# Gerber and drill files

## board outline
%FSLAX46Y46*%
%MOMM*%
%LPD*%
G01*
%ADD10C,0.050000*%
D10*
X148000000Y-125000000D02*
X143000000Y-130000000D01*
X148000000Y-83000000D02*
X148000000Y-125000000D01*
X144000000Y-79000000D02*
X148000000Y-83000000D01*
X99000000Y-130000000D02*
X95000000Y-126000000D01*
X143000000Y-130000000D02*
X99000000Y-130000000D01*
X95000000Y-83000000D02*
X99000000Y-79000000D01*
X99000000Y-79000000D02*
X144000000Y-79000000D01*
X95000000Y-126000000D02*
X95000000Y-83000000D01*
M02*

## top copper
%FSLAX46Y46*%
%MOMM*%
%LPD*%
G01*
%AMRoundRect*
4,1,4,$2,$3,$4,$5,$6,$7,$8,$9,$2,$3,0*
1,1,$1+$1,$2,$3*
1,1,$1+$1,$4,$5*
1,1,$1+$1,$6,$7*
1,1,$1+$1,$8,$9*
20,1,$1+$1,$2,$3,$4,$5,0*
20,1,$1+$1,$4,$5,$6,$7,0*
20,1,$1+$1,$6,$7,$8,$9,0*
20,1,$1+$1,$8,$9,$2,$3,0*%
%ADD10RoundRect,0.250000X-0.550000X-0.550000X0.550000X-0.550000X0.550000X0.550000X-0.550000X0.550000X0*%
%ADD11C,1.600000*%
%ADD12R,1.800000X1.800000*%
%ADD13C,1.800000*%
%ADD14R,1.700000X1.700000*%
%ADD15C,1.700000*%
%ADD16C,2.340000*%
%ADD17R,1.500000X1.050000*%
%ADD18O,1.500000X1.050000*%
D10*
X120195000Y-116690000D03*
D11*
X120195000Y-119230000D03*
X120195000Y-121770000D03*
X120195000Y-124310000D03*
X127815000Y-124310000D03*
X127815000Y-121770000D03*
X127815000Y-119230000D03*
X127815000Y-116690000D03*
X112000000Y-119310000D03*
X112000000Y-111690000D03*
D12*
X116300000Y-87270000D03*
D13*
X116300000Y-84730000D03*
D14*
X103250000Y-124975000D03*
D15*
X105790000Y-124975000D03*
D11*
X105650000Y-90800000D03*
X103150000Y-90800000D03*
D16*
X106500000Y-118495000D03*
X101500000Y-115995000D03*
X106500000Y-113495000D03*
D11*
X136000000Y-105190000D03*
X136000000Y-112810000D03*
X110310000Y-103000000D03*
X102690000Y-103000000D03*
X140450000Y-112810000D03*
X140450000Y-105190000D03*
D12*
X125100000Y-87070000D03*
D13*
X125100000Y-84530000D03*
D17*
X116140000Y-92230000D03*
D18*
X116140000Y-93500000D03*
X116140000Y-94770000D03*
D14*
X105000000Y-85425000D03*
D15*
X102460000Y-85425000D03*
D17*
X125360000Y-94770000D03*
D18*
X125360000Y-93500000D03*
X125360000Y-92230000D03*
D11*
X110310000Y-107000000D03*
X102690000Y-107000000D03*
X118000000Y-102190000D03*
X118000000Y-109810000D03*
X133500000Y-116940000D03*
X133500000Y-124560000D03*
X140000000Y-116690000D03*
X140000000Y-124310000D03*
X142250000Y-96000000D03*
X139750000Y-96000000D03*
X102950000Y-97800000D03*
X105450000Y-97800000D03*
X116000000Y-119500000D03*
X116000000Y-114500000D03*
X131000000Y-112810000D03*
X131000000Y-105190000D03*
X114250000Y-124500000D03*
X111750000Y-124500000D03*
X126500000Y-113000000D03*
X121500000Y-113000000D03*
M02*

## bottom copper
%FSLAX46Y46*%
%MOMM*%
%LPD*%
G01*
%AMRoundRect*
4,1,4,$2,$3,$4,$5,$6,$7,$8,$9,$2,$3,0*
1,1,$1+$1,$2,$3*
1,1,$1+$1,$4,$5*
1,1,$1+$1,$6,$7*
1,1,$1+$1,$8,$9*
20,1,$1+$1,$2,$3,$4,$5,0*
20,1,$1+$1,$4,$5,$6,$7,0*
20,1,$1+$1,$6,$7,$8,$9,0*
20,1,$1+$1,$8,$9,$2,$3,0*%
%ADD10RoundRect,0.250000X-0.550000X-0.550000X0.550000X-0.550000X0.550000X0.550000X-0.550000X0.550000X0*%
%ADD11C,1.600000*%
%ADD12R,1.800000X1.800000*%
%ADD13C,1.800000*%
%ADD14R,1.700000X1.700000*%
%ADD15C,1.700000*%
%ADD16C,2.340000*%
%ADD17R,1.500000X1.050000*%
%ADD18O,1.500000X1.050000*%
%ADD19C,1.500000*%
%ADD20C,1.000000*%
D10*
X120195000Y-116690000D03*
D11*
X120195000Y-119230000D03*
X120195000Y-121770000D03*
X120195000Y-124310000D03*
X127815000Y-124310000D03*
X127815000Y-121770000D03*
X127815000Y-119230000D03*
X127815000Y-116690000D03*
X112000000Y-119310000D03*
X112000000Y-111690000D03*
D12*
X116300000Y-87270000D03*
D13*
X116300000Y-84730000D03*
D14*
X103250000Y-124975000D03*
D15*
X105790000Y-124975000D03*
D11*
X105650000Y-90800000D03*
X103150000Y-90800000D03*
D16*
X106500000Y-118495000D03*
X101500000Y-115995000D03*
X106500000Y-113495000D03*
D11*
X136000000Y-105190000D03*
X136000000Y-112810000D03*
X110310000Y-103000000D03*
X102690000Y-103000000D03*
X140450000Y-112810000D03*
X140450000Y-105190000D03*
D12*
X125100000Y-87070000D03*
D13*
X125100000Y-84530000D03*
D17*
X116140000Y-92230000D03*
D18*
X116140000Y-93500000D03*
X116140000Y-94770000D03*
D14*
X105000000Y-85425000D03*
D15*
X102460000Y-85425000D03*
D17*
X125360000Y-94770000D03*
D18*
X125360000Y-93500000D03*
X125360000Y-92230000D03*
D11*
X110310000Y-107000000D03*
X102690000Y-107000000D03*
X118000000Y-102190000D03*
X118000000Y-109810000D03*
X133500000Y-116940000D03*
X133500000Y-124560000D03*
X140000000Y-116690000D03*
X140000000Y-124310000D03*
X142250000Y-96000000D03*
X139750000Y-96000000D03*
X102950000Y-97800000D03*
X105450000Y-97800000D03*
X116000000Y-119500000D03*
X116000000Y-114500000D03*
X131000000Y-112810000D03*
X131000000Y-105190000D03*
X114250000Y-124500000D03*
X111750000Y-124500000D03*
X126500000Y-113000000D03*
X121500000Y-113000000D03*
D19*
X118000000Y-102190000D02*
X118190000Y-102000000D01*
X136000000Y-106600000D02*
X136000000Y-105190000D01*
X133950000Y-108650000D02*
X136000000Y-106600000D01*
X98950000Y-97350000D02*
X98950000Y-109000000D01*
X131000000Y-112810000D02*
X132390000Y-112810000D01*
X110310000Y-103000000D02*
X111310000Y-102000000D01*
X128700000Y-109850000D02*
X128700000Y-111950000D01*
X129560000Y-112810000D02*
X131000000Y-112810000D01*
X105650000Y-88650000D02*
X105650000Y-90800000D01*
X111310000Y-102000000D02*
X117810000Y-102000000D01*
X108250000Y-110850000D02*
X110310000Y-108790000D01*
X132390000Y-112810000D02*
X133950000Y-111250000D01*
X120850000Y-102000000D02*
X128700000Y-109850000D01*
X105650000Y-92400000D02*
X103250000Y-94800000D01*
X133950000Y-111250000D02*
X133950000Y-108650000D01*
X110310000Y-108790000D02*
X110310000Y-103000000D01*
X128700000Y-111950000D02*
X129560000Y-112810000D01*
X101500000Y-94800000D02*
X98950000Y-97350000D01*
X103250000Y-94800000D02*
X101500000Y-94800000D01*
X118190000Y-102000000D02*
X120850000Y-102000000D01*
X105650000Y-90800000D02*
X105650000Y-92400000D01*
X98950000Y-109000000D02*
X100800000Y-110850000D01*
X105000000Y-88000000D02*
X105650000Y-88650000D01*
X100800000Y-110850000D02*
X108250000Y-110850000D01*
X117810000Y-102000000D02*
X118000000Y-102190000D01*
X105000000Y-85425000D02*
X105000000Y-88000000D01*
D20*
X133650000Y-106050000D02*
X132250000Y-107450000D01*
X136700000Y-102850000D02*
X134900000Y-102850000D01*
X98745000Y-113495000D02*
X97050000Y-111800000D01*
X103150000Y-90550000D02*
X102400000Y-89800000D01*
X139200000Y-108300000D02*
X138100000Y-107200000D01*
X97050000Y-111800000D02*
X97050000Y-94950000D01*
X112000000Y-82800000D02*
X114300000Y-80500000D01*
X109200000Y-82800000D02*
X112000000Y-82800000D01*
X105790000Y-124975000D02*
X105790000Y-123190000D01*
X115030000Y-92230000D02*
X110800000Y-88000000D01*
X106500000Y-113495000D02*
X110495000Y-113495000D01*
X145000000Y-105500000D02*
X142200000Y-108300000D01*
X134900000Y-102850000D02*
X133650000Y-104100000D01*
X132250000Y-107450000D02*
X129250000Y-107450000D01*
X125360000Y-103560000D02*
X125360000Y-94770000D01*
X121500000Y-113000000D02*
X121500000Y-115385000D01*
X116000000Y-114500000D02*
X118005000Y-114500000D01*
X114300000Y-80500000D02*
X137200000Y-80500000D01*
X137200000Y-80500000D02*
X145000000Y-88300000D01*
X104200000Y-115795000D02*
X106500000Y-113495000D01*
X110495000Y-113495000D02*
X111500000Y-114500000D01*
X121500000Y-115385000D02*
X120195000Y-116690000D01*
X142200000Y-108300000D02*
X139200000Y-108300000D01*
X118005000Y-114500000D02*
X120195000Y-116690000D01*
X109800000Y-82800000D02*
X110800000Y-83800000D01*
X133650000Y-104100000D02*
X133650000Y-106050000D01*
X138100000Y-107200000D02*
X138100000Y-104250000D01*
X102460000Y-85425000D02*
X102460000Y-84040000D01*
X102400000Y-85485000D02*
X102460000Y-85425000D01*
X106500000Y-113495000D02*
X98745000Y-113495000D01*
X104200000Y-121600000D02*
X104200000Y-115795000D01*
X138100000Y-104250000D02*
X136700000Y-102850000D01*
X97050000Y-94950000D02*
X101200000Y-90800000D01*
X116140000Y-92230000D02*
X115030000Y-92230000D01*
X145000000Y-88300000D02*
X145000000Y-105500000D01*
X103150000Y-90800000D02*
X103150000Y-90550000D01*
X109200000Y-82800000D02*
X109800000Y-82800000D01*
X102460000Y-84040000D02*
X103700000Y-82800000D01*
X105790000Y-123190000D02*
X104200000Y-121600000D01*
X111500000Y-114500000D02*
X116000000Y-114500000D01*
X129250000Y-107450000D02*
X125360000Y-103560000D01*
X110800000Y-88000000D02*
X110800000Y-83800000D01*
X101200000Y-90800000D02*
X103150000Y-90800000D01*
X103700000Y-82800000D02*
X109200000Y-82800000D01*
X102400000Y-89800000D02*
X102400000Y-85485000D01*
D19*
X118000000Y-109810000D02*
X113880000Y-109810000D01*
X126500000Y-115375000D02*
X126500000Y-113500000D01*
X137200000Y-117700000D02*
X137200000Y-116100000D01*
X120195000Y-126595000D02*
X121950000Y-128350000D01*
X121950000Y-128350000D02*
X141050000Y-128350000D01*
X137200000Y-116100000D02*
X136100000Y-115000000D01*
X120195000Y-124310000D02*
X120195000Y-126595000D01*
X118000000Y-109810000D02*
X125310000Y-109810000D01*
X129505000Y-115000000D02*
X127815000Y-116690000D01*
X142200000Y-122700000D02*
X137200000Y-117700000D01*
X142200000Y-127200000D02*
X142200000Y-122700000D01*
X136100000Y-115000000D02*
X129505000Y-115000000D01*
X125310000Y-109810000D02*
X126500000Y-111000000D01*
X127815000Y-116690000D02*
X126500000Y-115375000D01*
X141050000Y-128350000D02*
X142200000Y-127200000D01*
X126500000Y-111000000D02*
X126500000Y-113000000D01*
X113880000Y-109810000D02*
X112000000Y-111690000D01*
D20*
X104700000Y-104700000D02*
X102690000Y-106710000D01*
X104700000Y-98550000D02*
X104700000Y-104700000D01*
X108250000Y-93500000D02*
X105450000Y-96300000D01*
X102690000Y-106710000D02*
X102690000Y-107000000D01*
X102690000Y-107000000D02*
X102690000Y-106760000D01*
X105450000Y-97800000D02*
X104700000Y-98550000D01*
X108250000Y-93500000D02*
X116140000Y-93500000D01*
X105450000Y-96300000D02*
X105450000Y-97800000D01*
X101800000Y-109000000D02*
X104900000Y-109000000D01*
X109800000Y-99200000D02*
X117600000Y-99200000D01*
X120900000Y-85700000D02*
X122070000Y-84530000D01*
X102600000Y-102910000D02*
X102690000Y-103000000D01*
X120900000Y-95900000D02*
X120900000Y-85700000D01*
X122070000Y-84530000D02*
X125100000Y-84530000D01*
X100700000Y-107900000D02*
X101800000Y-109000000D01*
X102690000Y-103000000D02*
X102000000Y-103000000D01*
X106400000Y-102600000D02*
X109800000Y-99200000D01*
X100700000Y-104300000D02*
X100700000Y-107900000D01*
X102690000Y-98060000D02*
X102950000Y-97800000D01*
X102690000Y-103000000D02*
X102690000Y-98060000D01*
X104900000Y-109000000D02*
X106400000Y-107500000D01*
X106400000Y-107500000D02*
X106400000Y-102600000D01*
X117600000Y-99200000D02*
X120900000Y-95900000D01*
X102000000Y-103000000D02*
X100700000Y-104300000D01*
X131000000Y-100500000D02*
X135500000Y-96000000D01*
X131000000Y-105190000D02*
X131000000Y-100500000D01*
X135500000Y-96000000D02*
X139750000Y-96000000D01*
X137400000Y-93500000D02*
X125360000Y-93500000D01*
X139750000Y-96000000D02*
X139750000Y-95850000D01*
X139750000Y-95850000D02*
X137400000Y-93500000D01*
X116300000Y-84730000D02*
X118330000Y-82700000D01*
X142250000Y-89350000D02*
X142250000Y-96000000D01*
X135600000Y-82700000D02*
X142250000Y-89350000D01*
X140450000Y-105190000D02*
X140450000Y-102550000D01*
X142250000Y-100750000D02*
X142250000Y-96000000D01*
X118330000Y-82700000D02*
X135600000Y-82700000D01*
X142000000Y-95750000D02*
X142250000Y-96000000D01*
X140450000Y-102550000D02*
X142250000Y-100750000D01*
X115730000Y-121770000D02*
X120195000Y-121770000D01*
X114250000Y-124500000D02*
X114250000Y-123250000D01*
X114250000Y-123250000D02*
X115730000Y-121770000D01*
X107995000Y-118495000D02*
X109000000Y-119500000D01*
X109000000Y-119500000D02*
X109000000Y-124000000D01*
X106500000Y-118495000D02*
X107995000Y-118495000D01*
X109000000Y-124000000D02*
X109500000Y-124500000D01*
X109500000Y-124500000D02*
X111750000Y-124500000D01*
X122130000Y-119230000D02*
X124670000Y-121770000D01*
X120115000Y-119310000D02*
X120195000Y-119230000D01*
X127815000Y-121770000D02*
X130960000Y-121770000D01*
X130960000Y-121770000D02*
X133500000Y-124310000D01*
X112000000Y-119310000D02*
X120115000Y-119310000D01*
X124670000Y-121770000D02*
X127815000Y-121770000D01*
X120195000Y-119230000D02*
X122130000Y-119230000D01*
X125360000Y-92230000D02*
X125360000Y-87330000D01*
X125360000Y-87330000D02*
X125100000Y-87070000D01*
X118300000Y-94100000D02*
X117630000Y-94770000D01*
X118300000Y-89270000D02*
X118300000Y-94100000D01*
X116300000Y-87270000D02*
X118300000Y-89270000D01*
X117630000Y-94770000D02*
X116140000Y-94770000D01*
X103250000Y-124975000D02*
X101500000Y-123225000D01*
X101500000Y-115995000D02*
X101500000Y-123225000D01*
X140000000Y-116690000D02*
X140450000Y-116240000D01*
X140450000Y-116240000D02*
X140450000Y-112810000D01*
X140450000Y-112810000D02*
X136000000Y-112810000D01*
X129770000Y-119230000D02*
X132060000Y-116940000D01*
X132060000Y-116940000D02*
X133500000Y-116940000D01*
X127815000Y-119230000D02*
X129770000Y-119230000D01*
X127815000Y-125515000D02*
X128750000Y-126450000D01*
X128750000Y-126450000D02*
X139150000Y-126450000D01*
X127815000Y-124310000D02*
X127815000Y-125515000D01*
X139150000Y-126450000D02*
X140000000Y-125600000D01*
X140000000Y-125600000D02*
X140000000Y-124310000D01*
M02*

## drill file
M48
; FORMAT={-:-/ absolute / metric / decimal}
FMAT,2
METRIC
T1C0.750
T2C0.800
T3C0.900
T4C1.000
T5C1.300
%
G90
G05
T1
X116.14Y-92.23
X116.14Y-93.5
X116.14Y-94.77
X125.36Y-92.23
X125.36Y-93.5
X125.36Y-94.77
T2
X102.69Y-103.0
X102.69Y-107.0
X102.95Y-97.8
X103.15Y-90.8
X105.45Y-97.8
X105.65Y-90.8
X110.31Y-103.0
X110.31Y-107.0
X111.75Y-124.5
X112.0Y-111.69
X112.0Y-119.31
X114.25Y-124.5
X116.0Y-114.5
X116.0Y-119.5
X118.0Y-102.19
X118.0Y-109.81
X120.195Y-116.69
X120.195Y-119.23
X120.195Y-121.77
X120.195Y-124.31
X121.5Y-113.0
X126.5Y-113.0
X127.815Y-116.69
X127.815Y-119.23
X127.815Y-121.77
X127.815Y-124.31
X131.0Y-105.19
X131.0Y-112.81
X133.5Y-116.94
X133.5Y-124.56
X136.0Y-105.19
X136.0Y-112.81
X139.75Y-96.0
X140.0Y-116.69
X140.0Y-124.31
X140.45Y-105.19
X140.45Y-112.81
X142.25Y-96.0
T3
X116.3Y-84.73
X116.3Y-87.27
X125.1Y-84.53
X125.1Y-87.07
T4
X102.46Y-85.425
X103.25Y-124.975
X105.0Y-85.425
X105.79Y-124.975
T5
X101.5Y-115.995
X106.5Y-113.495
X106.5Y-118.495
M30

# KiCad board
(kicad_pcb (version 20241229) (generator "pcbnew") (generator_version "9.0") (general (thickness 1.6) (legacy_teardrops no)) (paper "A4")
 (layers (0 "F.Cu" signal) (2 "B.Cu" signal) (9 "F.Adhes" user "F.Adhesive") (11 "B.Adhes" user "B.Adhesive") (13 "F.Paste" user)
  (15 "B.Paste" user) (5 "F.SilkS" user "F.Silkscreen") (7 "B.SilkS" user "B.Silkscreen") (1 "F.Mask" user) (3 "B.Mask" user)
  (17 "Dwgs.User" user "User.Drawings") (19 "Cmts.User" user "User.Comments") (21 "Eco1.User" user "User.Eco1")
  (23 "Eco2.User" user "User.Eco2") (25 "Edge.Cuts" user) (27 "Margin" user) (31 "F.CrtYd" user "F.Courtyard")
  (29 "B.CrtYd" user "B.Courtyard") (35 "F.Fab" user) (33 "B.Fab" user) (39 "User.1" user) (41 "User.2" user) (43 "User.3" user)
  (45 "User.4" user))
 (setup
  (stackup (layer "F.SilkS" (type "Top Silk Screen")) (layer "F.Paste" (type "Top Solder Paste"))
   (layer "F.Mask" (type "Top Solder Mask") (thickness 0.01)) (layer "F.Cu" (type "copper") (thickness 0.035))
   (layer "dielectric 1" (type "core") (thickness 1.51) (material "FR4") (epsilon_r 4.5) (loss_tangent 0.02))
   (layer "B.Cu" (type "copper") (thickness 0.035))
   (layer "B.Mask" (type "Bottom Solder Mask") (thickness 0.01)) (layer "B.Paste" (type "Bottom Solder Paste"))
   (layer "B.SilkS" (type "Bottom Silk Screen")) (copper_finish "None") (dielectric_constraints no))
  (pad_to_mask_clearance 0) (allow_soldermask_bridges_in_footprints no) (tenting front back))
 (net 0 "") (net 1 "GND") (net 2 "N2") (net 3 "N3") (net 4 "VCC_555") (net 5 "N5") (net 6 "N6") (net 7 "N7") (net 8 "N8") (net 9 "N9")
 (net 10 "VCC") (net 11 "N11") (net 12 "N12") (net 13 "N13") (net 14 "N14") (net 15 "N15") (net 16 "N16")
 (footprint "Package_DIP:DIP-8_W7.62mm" (layer "F.Cu") (at 120.195 116.69)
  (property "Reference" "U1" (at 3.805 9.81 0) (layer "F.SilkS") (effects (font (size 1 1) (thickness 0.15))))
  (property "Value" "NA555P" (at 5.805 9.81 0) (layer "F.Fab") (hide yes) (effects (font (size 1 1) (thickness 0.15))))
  (pad "1" thru_hole roundrect (at 0 0) (size 1.6 1.6) (drill 0.8) (layers "*.Cu" "*.Mask") (remove_unused_layers no)
   (roundrect_rratio 0.15625) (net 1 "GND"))
  (pad "2" thru_hole circle (at 0 2.54) (size 1.6 1.6) (drill 0.8) (layers "*.Cu" "*.Mask") (remove_unused_layers no) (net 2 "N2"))
  (pad "3" thru_hole circle (at 0 5.08) (size 1.6 1.6) (drill 0.8) (layers "*.Cu" "*.Mask") (remove_unused_layers no) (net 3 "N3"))
  (pad "4" thru_hole circle (at 0 7.62) (size 1.6 1.6) (drill 0.8) (layers "*.Cu" "*.Mask") (remove_unused_layers no) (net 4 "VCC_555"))
  (pad "5" thru_hole circle (at 7.62 7.62) (size 1.6 1.6) (drill 0.8) (layers "*.Cu" "*.Mask") (remove_unused_layers no) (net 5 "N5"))
  (pad "6" thru_hole circle (at 7.62 5.08) (size 1.6 1.6) (drill 0.8) (layers "*.Cu" "*.Mask") (remove_unused_layers no) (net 2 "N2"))
  (pad "7" thru_hole circle (at 7.62 2.54) (size 1.6 1.6) (drill 0.8) (layers "*.Cu" "*.Mask") (remove_unused_layers no) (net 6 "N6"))
  (pad "8" thru_hole circle (at 7.62 0) (size 1.6 1.6) (drill 0.8) (layers "*.Cu" "*.Mask") (remove_unused_layers no) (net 4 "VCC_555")))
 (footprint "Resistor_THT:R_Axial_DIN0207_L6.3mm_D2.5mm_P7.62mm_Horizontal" (layer "F.Cu") (at 112 119.31 90)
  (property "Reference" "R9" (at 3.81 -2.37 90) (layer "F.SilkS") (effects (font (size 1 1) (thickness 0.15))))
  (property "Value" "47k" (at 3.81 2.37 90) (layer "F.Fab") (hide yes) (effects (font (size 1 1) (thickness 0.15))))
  (pad "1" thru_hole circle (at 0 0 90) (size 1.6 1.6) (drill 0.8) (layers "*.Cu" "*.Mask") (remove_unused_layers no) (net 2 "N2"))
  (pad "2" thru_hole circle (at 7.62 0 90) (size 1.6 1.6) (drill 0.8) (layers "*.Cu" "*.Mask") (remove_unused_layers no) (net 4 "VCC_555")))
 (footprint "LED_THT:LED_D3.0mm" (layer "F.Cu") (at 116.3 87.27 90)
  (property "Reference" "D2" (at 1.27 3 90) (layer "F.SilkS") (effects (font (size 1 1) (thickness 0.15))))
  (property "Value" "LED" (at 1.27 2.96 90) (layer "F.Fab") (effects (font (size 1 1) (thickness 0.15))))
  (pad "1" thru_hole rect (at 0 0 90) (size 1.8 1.8) (drill 0.9) (layers "*.Cu" "*.Mask") (remove_unused_layers no) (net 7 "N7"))
  (pad "2" thru_hole circle (at 2.54 0 90) (size 1.8 1.8) (drill 0.9) (layers "*.Cu" "*.Mask") (remove_unused_layers no) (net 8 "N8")))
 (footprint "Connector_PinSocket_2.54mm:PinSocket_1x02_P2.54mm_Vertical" (layer "F.Cu") (at 103.25 124.975 90)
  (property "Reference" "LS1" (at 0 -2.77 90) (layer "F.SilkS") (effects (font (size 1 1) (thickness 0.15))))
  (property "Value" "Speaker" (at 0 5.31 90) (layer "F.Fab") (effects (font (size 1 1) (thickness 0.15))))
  (pad "1" thru_hole rect (at 0 0 90) (size 1.7 1.7) (drill 1) (layers "*.Cu" "*.Mask") (remove_unused_layers no) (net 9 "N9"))
  (pad "2" thru_hole circle (at 0 2.54 90) (size 1.7 1.7) (drill 1) (layers "*.Cu" "*.Mask") (remove_unused_layers no) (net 1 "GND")))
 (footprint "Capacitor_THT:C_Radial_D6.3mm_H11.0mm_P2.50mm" (layer "F.Cu") (at 105.65 90.8 180)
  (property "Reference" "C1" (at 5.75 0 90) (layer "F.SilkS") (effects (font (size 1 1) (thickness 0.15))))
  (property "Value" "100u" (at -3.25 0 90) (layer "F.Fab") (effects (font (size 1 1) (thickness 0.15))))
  (pad "1" thru_hole circle (at 0 0 180) (size 1.6 1.6) (drill 0.8) (layers "*.Cu" "*.Mask") (remove_unused_layers no) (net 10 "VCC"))
  (pad "2" thru_hole circle (at 2.5 0 180) (size 1.6 1.6) (drill 0.8) (layers "*.Cu" "*.Mask") (remove_unused_layers no) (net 1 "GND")))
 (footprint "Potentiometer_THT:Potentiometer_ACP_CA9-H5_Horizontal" (layer "F.Cu") (at 106.5 118.495 180)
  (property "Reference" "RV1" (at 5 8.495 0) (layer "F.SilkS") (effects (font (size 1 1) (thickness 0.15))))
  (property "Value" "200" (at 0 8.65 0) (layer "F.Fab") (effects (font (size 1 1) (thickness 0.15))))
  (pad "1" thru_hole circle (at 0 0 180) (size 2.34 2.34) (drill 1.3) (layers "*.Cu" "*.Mask") (remove_unused_layers no) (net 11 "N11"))
  (pad "2" thru_hole circle (at 5 2.5 180) (size 2.34 2.34) (drill 1.3) (layers "*.Cu" "*.Mask") (remove_unused_layers no) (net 9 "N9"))
  (pad "3" thru_hole circle (at 0 5 180) (size 2.34 2.34) (drill 1.3) (layers "*.Cu" "*.Mask") (remove_unused_layers no) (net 1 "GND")))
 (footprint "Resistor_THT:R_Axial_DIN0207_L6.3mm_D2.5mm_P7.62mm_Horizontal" (layer "F.Cu") (at 136 105.19 -90)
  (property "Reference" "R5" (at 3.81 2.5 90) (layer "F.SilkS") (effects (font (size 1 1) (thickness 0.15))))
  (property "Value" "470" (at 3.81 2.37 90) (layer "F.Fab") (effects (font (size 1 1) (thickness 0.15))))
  (pad "1" thru_hole circle (at 0 0 270) (size 1.6 1.6) (drill 0.8) (layers "*.Cu" "*.Mask") (remove_unused_layers no) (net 10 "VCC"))
  (pad "2" thru_hole circle (at 7.62 0 270) (size 1.6 1.6) (drill 0.8) (layers "*.Cu" "*.Mask") (remove_unused_layers no) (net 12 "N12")))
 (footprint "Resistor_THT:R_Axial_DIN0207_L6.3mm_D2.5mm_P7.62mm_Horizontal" (layer "F.Cu") (at 110.31 103 180)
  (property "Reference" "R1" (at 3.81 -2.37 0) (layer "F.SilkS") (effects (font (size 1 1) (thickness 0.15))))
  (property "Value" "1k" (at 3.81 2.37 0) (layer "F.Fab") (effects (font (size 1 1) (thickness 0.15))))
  (pad "1" thru_hole circle (at 0 0 180) (size 1.6 1.6) (drill 0.8) (layers "*.Cu" "*.Mask") (remove_unused_layers no) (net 10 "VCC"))
  (pad "2" thru_hole circle (at 7.62 0 180) (size 1.6 1.6) (drill 0.8) (layers "*.Cu" "*.Mask") (remove_unused_layers no) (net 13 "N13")))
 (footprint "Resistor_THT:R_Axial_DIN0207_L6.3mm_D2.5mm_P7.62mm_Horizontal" (layer "F.Cu") (at 140.45 112.81 90)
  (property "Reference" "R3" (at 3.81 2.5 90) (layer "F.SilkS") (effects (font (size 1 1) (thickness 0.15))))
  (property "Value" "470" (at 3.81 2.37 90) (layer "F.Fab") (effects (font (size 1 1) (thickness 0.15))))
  (pad "1" thru_hole circle (at 0 0 90) (size 1.6 1.6) (drill 0.8) (layers "*.Cu" "*.Mask") (remove_unused_layers no) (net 12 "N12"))
  (pad "2" thru_hole circle (at 7.62 0 90) (size 1.6 1.6) (drill 0.8) (layers "*.Cu" "*.Mask") (remove_unused_layers no) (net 8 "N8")))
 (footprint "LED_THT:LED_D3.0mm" (layer "F.Cu") (at 125.1 87.07 90)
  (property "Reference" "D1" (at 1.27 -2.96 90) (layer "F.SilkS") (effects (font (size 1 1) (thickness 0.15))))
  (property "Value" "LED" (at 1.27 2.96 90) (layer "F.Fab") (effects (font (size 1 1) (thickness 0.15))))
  (pad "1" thru_hole rect (at 0 0 90) (size 1.8 1.8) (drill 0.9) (layers "*.Cu" "*.Mask") (remove_unused_layers no) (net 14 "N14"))
  (pad "2" thru_hole circle (at 2.54 0 90) (size 1.8 1.8) (drill 0.9) (layers "*.Cu" "*.Mask") (remove_unused_layers no) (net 13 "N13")))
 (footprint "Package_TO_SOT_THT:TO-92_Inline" (layer "F.Cu") (at 116.14 92.23 -90)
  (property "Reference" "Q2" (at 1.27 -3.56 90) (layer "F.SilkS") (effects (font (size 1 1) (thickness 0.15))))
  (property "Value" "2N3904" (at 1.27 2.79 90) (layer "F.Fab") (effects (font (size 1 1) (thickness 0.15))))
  (pad "1" thru_hole rect (at 0 0 270) (size 1.05 1.5) (drill 0.75) (layers "*.Cu" "*.Mask") (remove_unused_layers no) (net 1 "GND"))
  (pad "2" thru_hole oval (at 1.27 0 270) (size 1.05 1.5) (drill 0.75) (layers "*.Cu" "*.Mask") (remove_unused_layers no) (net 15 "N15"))
  (pad "3" thru_hole oval (at 2.54 0 270) (size 1.05 1.5) (drill 0.75) (layers "*.Cu" "*.Mask") (remove_unused_layers no) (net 7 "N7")))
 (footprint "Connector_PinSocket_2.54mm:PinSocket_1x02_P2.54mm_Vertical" (layer "F.Cu") (at 105 85.425 -90)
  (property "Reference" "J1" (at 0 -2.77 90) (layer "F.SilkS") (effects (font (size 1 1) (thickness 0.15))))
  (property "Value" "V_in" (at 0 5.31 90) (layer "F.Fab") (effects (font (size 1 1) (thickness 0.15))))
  (pad "1" thru_hole rect (at 0 0 270) (size 1.7 1.7) (drill 1) (layers "*.Cu" "*.Mask") (remove_unused_layers no) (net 10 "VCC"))
  (pad "2" thru_hole circle (at 0 2.54 270) (size 1.7 1.7) (drill 1) (layers "*.Cu" "*.Mask") (remove_unused_layers no) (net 1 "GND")))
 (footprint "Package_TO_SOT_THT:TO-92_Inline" (layer "F.Cu") (at 125.36 94.77 90)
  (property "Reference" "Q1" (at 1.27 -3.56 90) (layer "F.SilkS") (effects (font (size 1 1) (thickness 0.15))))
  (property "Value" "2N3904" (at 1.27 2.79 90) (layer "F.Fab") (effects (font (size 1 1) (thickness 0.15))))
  (pad "1" thru_hole rect (at 0 0 90) (size 1.05 1.5) (drill 0.75) (layers "*.Cu" "*.Mask") (remove_unused_layers no) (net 1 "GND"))
  (pad "2" thru_hole oval (at 1.27 0 90) (size 1.05 1.5) (drill 0.75) (layers "*.Cu" "*.Mask") (remove_unused_layers no) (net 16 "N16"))
  (pad "3" thru_hole oval (at 2.54 0 90) (size 1.05 1.5) (drill 0.75) (layers "*.Cu" "*.Mask") (remove_unused_layers no) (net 14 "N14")))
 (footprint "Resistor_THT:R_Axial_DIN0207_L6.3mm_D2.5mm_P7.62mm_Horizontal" (layer "F.Cu") (at 110.31 107 180)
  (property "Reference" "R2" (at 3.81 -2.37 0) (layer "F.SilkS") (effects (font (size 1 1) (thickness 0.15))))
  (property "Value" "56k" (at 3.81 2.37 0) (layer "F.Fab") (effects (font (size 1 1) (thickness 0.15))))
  (pad "1" thru_hole circle (at 0 0 180) (size 1.6 1.6) (drill 0.8) (layers "*.Cu" "*.Mask") (remove_unused_layers no) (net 10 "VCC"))
  (pad "2" thru_hole circle (at 7.62 0 180) (size 1.6 1.6) (drill 0.8) (layers "*.Cu" "*.Mask") (remove_unused_layers no) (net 15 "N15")))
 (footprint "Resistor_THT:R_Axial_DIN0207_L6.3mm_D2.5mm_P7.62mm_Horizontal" (layer "F.Cu") (at 118 102.19 -90)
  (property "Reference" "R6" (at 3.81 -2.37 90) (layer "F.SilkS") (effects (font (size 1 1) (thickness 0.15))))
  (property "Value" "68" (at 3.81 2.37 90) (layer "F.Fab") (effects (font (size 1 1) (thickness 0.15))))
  (pad "1" thru_hole circle (at 0 0 270) (size 1.6 1.6) (drill 0.8) (layers "*.Cu" "*.Mask") (remove_unused_layers no) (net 10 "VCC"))
  (pad "2" thru_hole circle (at 7.62 0 270) (size 1.6 1.6) (drill 0.8) (layers "*.Cu" "*.Mask") (remove_unused_layers no) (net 4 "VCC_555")))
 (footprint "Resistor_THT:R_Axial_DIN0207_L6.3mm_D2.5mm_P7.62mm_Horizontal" (layer "F.Cu") (at 133.5 116.94 -90)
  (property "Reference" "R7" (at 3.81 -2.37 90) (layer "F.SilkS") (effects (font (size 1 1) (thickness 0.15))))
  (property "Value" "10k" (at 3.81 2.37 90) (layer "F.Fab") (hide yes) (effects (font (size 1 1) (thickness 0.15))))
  (pad "1" thru_hole circle (at 0 0 270) (size 1.6 1.6) (drill 0.8) (layers "*.Cu" "*.Mask") (remove_unused_layers no) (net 6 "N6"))
  (pad "2" thru_hole circle (at 7.62 0 270) (size 1.6 1.6) (drill 0.8) (layers "*.Cu" "*.Mask") (remove_unused_layers no) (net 2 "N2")))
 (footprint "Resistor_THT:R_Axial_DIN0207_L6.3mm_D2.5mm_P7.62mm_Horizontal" (layer "F.Cu") (at 140 116.69 -90)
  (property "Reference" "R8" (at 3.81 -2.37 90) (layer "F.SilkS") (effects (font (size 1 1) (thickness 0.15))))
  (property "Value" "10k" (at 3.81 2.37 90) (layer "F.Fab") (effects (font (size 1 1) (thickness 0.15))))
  (pad "1" thru_hole circle (at 0 0 270) (size 1.6 1.6) (drill 0.8) (layers "*.Cu" "*.Mask") (remove_unused_layers no) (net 12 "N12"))
  (pad "2" thru_hole circle (at 7.62 0 270) (size 1.6 1.6) (drill 0.8) (layers "*.Cu" "*.Mask") (remove_unused_layers no) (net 5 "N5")))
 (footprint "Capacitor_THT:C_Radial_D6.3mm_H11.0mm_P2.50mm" (layer "F.Cu") (at 142.25 96 180)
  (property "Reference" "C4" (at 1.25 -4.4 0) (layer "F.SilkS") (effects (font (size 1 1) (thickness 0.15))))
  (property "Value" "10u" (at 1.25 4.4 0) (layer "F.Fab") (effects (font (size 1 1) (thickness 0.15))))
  (pad "1" thru_hole circle (at 0 0 180) (size 1.6 1.6) (drill 0.8) (layers "*.Cu" "*.Mask") (remove_unused_layers no) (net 8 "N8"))
  (pad "2" thru_hole circle (at 2.5 0 180) (size 1.6 1.6) (drill 0.8) (layers "*.Cu" "*.Mask") (remove_unused_layers no) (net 16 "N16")))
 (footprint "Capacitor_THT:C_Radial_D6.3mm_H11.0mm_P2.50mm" (layer "F.Cu") (at 102.95 97.8)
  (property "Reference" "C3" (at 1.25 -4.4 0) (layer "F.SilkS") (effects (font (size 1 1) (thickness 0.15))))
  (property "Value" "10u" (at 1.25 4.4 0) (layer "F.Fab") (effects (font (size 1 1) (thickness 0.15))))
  (pad "1" thru_hole circle (at 0 0) (size 1.6 1.6) (drill 0.8) (layers "*.Cu" "*.Mask") (remove_unused_layers no) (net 13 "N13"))
  (pad "2" thru_hole circle (at 2.5 0) (size 1.6 1.6) (drill 0.8) (layers "*.Cu" "*.Mask") (remove_unused_layers no) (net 15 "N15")))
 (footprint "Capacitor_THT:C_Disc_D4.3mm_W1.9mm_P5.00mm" (layer "F.Cu") (at 116 119.5 90)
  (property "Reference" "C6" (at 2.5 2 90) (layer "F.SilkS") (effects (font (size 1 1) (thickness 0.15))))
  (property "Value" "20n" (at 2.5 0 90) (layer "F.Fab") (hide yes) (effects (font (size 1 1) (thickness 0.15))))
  (pad "1" thru_hole circle (at 0 0 90) (size 1.6 1.6) (drill 0.8) (layers "*.Cu" "*.Mask") (remove_unused_layers no) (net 2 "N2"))
  (pad "2" thru_hole circle (at 5 0 90) (size 1.6 1.6) (drill 0.8) (layers "*.Cu" "*.Mask") (remove_unused_layers no) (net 1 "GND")))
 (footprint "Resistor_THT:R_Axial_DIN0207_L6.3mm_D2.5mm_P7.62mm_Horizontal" (layer "F.Cu") (at 131 112.81 90)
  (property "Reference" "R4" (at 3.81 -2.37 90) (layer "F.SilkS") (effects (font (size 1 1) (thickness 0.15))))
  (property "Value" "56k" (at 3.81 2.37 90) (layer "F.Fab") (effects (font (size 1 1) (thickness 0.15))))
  (pad "1" thru_hole circle (at 0 0 90) (size 1.6 1.6) (drill 0.8) (layers "*.Cu" "*.Mask") (remove_unused_layers no) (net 10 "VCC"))
  (pad "2" thru_hole circle (at 7.62 0 90) (size 1.6 1.6) (drill 0.8) (layers "*.Cu" "*.Mask") (remove_unused_layers no) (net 16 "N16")))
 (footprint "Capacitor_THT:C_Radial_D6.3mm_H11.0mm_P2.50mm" (layer "F.Cu") (at 114.25 124.5 180)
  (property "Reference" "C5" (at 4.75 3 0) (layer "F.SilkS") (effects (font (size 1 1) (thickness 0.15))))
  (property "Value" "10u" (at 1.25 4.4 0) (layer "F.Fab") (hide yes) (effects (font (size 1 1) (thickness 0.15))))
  (pad "1" thru_hole circle (at 0 0 180) (size 1.6 1.6) (drill 0.8) (layers "*.Cu" "*.Mask") (remove_unused_layers no) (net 3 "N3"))
  (pad "2" thru_hole circle (at 2.5 0 180) (size 1.6 1.6) (drill 0.8) (layers "*.Cu" "*.Mask") (remove_unused_layers no) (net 11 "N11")))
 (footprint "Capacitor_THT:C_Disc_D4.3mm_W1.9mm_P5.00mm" (layer "F.Cu") (at 126.5 113 180)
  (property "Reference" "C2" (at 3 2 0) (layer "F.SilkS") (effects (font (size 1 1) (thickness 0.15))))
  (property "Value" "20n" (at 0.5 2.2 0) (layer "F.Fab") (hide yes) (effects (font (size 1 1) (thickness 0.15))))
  (pad "1" thru_hole circle (at 0 0 180) (size 1.6 1.6) (drill 0.8) (layers "*.Cu" "*.Mask") (remove_unused_layers no) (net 4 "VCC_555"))
  (pad "2" thru_hole circle (at 5 0 180) (size 1.6 1.6) (drill 0.8) (layers "*.Cu" "*.Mask") (remove_unused_layers no) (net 1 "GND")))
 (gr_line (start 148 125) (end 143 130) (stroke (width 0.05) (type default)) (layer "Edge.Cuts"))
 (gr_line (start 148 83) (end 148 125) (stroke (width 0.05) (type default)) (layer "Edge.Cuts"))
 (gr_line (start 144 79) (end 148 83) (stroke (width 0.05) (type default)) (layer "Edge.Cuts"))
 (gr_line (start 99 130) (end 95 126) (stroke (width 0.05) (type default)) (layer "Edge.Cuts"))
 (gr_line (start 143 130) (end 99 130) (stroke (width 0.05) (type default)) (layer "Edge.Cuts"))
 (gr_line (start 95 83) (end 99 79) (stroke (width 0.05) (type default)) (layer "Edge.Cuts"))
 (gr_line (start 99 79) (end 144 79) (stroke (width 0.05) (type default)) (layer "Edge.Cuts"))
 (gr_line (start 95 126) (end 95 83) (stroke (width 0.05) (type default)) (layer "Edge.Cuts"))
 (segment (start 118 102.19) (end 118.19 102) (width 1.5) (layer "B.Cu") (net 10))
 (segment (start 136 106.6) (end 136 105.19) (width 1.5) (layer "B.Cu") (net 10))
 (segment (start 133.95 108.65) (end 136 106.6) (width 1.5) (layer "B.Cu") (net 10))
 (segment (start 98.95 97.35) (end 98.95 109) (width 1.5) (layer "B.Cu") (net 10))
 (segment (start 131 112.81) (end 132.39 112.81) (width 1.5) (layer "B.Cu") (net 10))
 (segment (start 110.31 103) (end 111.31 102) (width 1.5) (layer "B.Cu") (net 10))
 (segment (start 128.7 109.85) (end 128.7 111.95) (width 1.5) (layer "B.Cu") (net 10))
 (segment (start 129.56 112.81) (end 131 112.81) (width 1.5) (layer "B.Cu") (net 10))
 (segment (start 105.65 88.65) (end 105.65 90.8) (width 1.5) (layer "B.Cu") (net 10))
 (segment (start 111.31 102) (end 117.81 102) (width 1.5) (layer "B.Cu") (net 10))
 (segment (start 108.25 110.85) (end 110.31 108.79) (width 1.5) (layer "B.Cu") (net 10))
 (segment (start 132.39 112.81) (end 133.95 111.25) (width 1.5) (layer "B.Cu") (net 10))
 (segment (start 120.85 102) (end 128.7 109.85) (width 1.5) (layer "B.Cu") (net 10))
 (segment (start 105.65 92.4) (end 103.25 94.8) (width 1.5) (layer "B.Cu") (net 10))
 (segment (start 133.95 111.25) (end 133.95 108.65) (width 1.5) (layer "B.Cu") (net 10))
 (segment (start 110.31 108.79) (end 110.31 103) (width 1.5) (layer "B.Cu") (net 10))
 (segment (start 128.7 111.95) (end 129.56 112.81) (width 1.5) (layer "B.Cu") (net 10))
 (segment (start 101.5 94.8) (end 98.95 97.35) (width 1.5) (layer "B.Cu") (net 10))
 (segment (start 103.25 94.8) (end 101.5 94.8) (width 1.5) (layer "B.Cu") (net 10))
 (segment (start 118.19 102) (end 120.85 102) (width 1.5) (layer "B.Cu") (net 10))
 (segment (start 105.65 90.8) (end 105.65 92.4) (width 1.5) (layer "B.Cu") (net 10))
 (segment (start 98.95 109) (end 100.8 110.85) (width 1.5) (layer "B.Cu") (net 10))
 (segment (start 105 88) (end 105.65 88.65) (width 1.5) (layer "B.Cu") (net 10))
 (segment (start 100.8 110.85) (end 108.25 110.85) (width 1.5) (layer "B.Cu") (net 10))
 (segment (start 117.81 102) (end 118 102.19) (width 1.5) (layer "B.Cu") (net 10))
 (segment (start 105 85.425) (end 105 88) (width 1.5) (layer "B.Cu") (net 10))
 (segment (start 133.65 106.05) (end 132.25 107.45) (width 1) (layer "B.Cu") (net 1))
 (segment (start 136.7 102.85) (end 134.9 102.85) (width 1) (layer "B.Cu") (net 1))
 (segment (start 98.745 113.495) (end 97.05 111.8) (width 1) (layer "B.Cu") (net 1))
 (segment (start 103.15 90.55) (end 102.4 89.8) (width 1) (layer "B.Cu") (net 1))
 (segment (start 139.2 108.3) (end 138.1 107.2) (width 1) (layer "B.Cu") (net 1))
 (segment (start 97.05 111.8) (end 97.05 94.95) (width 1) (layer "B.Cu") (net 1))
 (segment (start 112 82.8) (end 114.3 80.5) (width 1) (layer "B.Cu") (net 1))
 (segment (start 109.2 82.8) (end 112 82.8) (width 1) (layer "B.Cu") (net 1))
 (segment (start 105.79 124.975) (end 105.79 123.19) (width 1) (layer "B.Cu") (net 1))
 (segment (start 115.03 92.23) (end 110.8 88) (width 1) (layer "B.Cu") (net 1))
 (segment (start 106.5 113.495) (end 110.495 113.495) (width 1) (layer "B.Cu") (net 1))
 (segment (start 145 105.5) (end 142.2 108.3) (width 1) (layer "B.Cu") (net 1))
 (segment (start 134.9 102.85) (end 133.65 104.1) (width 1) (layer "B.Cu") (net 1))
 (segment (start 132.25 107.45) (end 129.25 107.45) (width 1) (layer "B.Cu") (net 1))
 (segment (start 125.36 103.56) (end 125.36 94.77) (width 1) (layer "B.Cu") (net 1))
 (segment (start 121.5 113) (end 121.5 115.385) (width 1) (layer "B.Cu") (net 1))
 (segment (start 116 114.5) (end 118.005 114.5) (width 1) (layer "B.Cu") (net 1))
 (segment (start 114.3 80.5) (end 137.2 80.5) (width 1) (layer "B.Cu") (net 1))
 (segment (start 137.2 80.5) (end 145 88.3) (width 1) (layer "B.Cu") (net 1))
 (segment (start 104.2 115.795) (end 106.5 113.495) (width 1) (layer "B.Cu") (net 1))
 (segment (start 110.495 113.495) (end 111.5 114.5) (width 1) (layer "B.Cu") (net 1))
 (segment (start 121.5 115.385) (end 120.195 116.69) (width 1) (layer "B.Cu") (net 1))
 (segment (start 142.2 108.3) (end 139.2 108.3) (width 1) (layer "B.Cu") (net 1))
 (segment (start 118.005 114.5) (end 120.195 116.69) (width 1) (layer "B.Cu") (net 1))
 (segment (start 109.8 82.8) (end 110.8 83.8) (width 1) (layer "B.Cu") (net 1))
 (segment (start 133.65 104.1) (end 133.65 106.05) (width 1) (layer "B.Cu") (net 1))
 (segment (start 138.1 107.2) (end 138.1 104.25) (width 1) (layer "B.Cu") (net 1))
 (segment (start 102.46 85.425) (end 102.46 84.04) (width 1) (layer "B.Cu") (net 1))
 (segment (start 102.4 85.485) (end 102.46 85.425) (width 1) (layer "B.Cu") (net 1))
 (segment (start 106.5 113.495) (end 98.745 113.495) (width 1) (layer "B.Cu") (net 1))
 (segment (start 104.2 121.6) (end 104.2 115.795) (width 1) (layer "B.Cu") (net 1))
 (segment (start 138.1 104.25) (end 136.7 102.85) (width 1) (layer "B.Cu") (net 1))
 (segment (start 97.05 94.95) (end 101.2 90.8) (width 1) (layer "B.Cu") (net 1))
 (segment (start 116.14 92.23) (end 115.03 92.23) (width 1) (layer "B.Cu") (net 1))
 (segment (start 145 88.3) (end 145 105.5) (width 1) (layer "B.Cu") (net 1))
 (segment (start 103.15 90.8) (end 103.15 90.55) (width 1) (layer "B.Cu") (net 1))
 (segment (start 109.2 82.8) (end 109.8 82.8) (width 1) (layer "B.Cu") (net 1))
 (segment (start 102.46 84.04) (end 103.7 82.8) (width 1) (layer "B.Cu") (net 1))
 (segment (start 105.79 123.19) (end 104.2 121.6) (width 1) (layer "B.Cu") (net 1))
 (segment (start 111.5 114.5) (end 116 114.5) (width 1) (layer "B.Cu") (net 1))
 (segment (start 129.25 107.45) (end 125.36 103.56) (width 1) (layer "B.Cu") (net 1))
 (segment (start 110.8 88) (end 110.8 83.8) (width 1) (layer "B.Cu") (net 1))
 (segment (start 101.2 90.8) (end 103.15 90.8) (width 1) (layer "B.Cu") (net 1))
 (segment (start 103.7 82.8) (end 109.2 82.8) (width 1) (layer "B.Cu") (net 1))
 (segment (start 102.4 89.8) (end 102.4 85.485) (width 1) (layer "B.Cu") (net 1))
 (segment (start 118 109.81) (end 113.88 109.81) (width 1.5) (layer "B.Cu") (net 4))
 (segment (start 126.5 115.375) (end 126.5 113.5) (width 1.5) (layer "B.Cu") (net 4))
 (segment (start 137.2 117.7) (end 137.2 116.1) (width 1.5) (layer "B.Cu") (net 4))
 (segment (start 120.195 126.595) (end 121.95 128.35) (width 1.5) (layer "B.Cu") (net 4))
 (segment (start 121.95 128.35) (end 141.05 128.35) (width 1.5) (layer "B.Cu") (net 4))
 (segment (start 137.2 116.1) (end 136.1 115) (width 1.5) (layer "B.Cu") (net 4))
 (segment (start 120.195 124.31) (end 120.195 126.595) (width 1.5) (layer "B.Cu") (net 4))
 (segment (start 118 109.81) (end 125.31 109.81) (width 1.5) (layer "B.Cu") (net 4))
 (segment (start 129.505 115) (end 127.815 116.69) (width 1.5) (layer "B.Cu") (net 4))
 (segment (start 142.2 122.7) (end 137.2 117.7) (width 1.5) (layer "B.Cu") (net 4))
 (segment (start 142.2 127.2) (end 142.2 122.7) (width 1.5) (layer "B.Cu") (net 4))
 (segment (start 136.1 115) (end 129.505 115) (width 1.5) (layer "B.Cu") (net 4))
 (segment (start 125.31 109.81) (end 126.5 111) (width 1.5) (layer "B.Cu") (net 4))
 (segment (start 127.815 116.69) (end 126.5 115.375) (width 1.5) (layer "B.Cu") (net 4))
 (segment (start 141.05 128.35) (end 142.2 127.2) (width 1.5) (layer "B.Cu") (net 4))
 (segment (start 126.5 111) (end 126.5 113) (width 1.5) (layer "B.Cu") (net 4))
 (segment (start 113.88 109.81) (end 112 111.69) (width 1.5) (layer "B.Cu") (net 4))
 (segment (start 104.7 104.7) (end 102.69 106.71) (width 1) (layer "B.Cu") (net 15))
 (segment (start 104.7 98.55) (end 104.7 104.7) (width 1) (layer "B.Cu") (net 15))
 (segment (start 108.25 93.5) (end 105.45 96.3) (width 1) (layer "B.Cu") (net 15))
 (segment (start 102.69 106.71) (end 102.69 107) (width 1) (layer "B.Cu") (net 15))
 (segment (start 102.69 107) (end 102.69 106.76) (width 1) (layer "B.Cu") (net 15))
 (segment (start 105.45 97.8) (end 104.7 98.55) (width 1) (layer "B.Cu") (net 15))
 (segment (start 108.25 93.5) (end 116.14 93.5) (width 1) (layer "B.Cu") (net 15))
 (segment (start 105.45 96.3) (end 105.45 97.8) (width 1) (layer "B.Cu") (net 15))
 (segment (start 101.8 109) (end 104.9 109) (width 1) (layer "B.Cu") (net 13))
 (segment (start 109.8 99.2) (end 117.6 99.2) (width 1) (layer "B.Cu") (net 13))
 (segment (start 120.9 85.7) (end 122.07 84.53) (width 1) (layer "B.Cu") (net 13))
 (segment (start 102.6 102.91) (end 102.69 103) (width 1) (layer "B.Cu") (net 13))
 (segment (start 120.9 95.9) (end 120.9 85.7) (width 1) (layer "B.Cu") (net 13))
 (segment (start 122.07 84.53) (end 125.1 84.53) (width 1) (layer "B.Cu") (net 13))
 (segment (start 100.7 107.9) (end 101.8 109) (width 1) (layer "B.Cu") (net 13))
 (segment (start 102.69 103) (end 102 103) (width 1) (layer "B.Cu") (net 13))
 (segment (start 106.4 102.6) (end 109.8 99.2) (width 1) (layer "B.Cu") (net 13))
 (segment (start 100.7 104.3) (end 100.7 107.9) (width 1) (layer "B.Cu") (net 13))
 (segment (start 102.69 98.06) (end 102.95 97.8) (width 1) (layer "B.Cu") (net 13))
 (segment (start 102.69 103) (end 102.69 98.06) (width 1) (layer "B.Cu") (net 13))
 (segment (start 104.9 109) (end 106.4 107.5) (width 1) (layer "B.Cu") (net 13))
 (segment (start 106.4 107.5) (end 106.4 102.6) (width 1) (layer "B.Cu") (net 13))
 (segment (start 117.6 99.2) (end 120.9 95.9) (width 1) (layer "B.Cu") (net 13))
 (segment (start 102 103) (end 100.7 104.3) (width 1) (layer "B.Cu") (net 13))
 (segment (start 131 100.5) (end 135.5 96) (width 1) (layer "B.Cu") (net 16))
 (segment (start 131 105.19) (end 131 100.5) (width 1) (layer "B.Cu") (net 16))
 (segment (start 135.5 96) (end 139.75 96) (width 1) (layer "B.Cu") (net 16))
 (segment (start 137.4 93.5) (end 125.36 93.5) (width 1) (layer "B.Cu") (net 16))
 (segment (start 139.75 96) (end 139.75 95.85) (width 1) (layer "B.Cu") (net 16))
 (segment (start 139.75 95.85) (end 137.4 93.5) (width 1) (layer "B.Cu") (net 16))
 (segment (start 116.3 84.73) (end 118.33 82.7) (width 1) (layer "B.Cu") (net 8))
 (segment (start 142.25 89.35) (end 142.25 96) (width 1) (layer "B.Cu") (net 8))
 (segment (start 135.6 82.7) (end 142.25 89.35) (width 1) (layer "B.Cu") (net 8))
 (segment (start 140.45 105.19) (end 140.45 102.55) (width 1) (layer "B.Cu") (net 8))
 (segment (start 142.25 100.75) (end 142.25 96) (width 1) (layer "B.Cu") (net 8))
 (segment (start 118.33 82.7) (end 135.6 82.7) (width 1) (layer "B.Cu") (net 8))
 (segment (start 142 95.75) (end 142.25 96) (width 1) (layer "B.Cu") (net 8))
 (segment (start 140.45 102.55) (end 142.25 100.75) (width 1) (layer "B.Cu") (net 8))
 (segment (start 115.73 121.77) (end 120.195 121.77) (width 1) (layer "B.Cu") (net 3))
 (segment (start 114.25 124.5) (end 114.25 123.25) (width 1) (layer "B.Cu") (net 3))
 (segment (start 114.25 123.25) (end 115.73 121.77) (width 1) (layer "B.Cu") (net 3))
 (segment (start 107.995 118.495) (end 109 119.5) (width 1) (layer "B.Cu") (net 11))
 (segment (start 109 119.5) (end 109 124) (width 1) (layer "B.Cu") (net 11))
 (segment (start 106.5 118.495) (end 107.995 118.495) (width 1) (layer "B.Cu") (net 11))
 (segment (start 109 124) (end 109.5 124.5) (width 1) (layer "B.Cu") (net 11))
 (segment (start 109.5 124.5) (end 111.75 124.5) (width 1) (layer "B.Cu") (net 11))
 (segment (start 122.13 119.23) (end 124.67 121.77) (width 1) (layer "B.Cu") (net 2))
 (segment (start 120.115 119.31) (end 120.195 119.23) (width 1) (layer "B.Cu") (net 2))
 (segment (start 127.815 121.77) (end 130.96 121.77) (width 1) (layer "B.Cu") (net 2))
 (segment (start 130.96 121.77) (end 133.5 124.31) (width 1) (layer "B.Cu") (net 2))
 (segment (start 112 119.31) (end 120.115 119.31) (width 1) (layer "B.Cu") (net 2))
 (segment (start 124.67 121.77) (end 127.815 121.77) (width 1) (layer "B.Cu") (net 2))
 (segment (start 120.195 119.23) (end 122.13 119.23) (width 1) (layer "B.Cu") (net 2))
 (segment (start 125.36 92.23) (end 125.36 87.33) (width 1) (layer "B.Cu") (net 14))
 (segment (start 125.36 87.33) (end 125.1 87.07) (width 1) (layer "B.Cu") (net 14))
 (segment (start 118.3 94.1) (end 117.63 94.77) (width 1) (layer "B.Cu") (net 7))
 (segment (start 118.3 89.27) (end 118.3 94.1) (width 1) (layer "B.Cu") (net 7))
 (segment (start 116.3 87.27) (end 118.3 89.27) (width 1) (layer "B.Cu") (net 7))
 (segment (start 117.63 94.77) (end 116.14 94.77) (width 1) (layer "B.Cu") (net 7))
 (segment (start 103.25 124.975) (end 101.5 123.225) (width 1) (layer "B.Cu") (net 9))
 (segment (start 101.5 115.995) (end 101.5 123.225) (width 1) (layer "B.Cu") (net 9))
 (segment (start 140 116.69) (end 140.45 116.24) (width 1) (layer "B.Cu") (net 12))
 (segment (start 140.45 116.24) (end 140.45 112.81) (width 1) (layer "B.Cu") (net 12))
 (segment (start 140.45 112.81) (end 136 112.81) (width 1) (layer "B.Cu") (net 12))
 (segment (start 129.77 119.23) (end 132.06 116.94) (width 1) (layer "B.Cu") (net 6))
 (segment (start 132.06 116.94) (end 133.5 116.94) (width 1) (layer "B.Cu") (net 6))
 (segment (start 127.815 119.23) (end 129.77 119.23) (width 1) (layer "B.Cu") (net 6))
 (segment (start 127.815 125.515) (end 128.75 126.45) (width 1) (layer "B.Cu") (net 5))
 (segment (start 128.75 126.45) (end 139.15 126.45) (width 1) (layer "B.Cu") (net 5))
 (segment (start 127.815 124.31) (end 127.815 125.515) (width 1) (layer "B.Cu") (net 5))
 (segment (start 139.15 126.45) (end 140 125.6) (width 1) (layer "B.Cu") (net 5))
 (segment (start 140 125.6) (end 140 124.31) (width 1) (layer "B.Cu") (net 5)))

